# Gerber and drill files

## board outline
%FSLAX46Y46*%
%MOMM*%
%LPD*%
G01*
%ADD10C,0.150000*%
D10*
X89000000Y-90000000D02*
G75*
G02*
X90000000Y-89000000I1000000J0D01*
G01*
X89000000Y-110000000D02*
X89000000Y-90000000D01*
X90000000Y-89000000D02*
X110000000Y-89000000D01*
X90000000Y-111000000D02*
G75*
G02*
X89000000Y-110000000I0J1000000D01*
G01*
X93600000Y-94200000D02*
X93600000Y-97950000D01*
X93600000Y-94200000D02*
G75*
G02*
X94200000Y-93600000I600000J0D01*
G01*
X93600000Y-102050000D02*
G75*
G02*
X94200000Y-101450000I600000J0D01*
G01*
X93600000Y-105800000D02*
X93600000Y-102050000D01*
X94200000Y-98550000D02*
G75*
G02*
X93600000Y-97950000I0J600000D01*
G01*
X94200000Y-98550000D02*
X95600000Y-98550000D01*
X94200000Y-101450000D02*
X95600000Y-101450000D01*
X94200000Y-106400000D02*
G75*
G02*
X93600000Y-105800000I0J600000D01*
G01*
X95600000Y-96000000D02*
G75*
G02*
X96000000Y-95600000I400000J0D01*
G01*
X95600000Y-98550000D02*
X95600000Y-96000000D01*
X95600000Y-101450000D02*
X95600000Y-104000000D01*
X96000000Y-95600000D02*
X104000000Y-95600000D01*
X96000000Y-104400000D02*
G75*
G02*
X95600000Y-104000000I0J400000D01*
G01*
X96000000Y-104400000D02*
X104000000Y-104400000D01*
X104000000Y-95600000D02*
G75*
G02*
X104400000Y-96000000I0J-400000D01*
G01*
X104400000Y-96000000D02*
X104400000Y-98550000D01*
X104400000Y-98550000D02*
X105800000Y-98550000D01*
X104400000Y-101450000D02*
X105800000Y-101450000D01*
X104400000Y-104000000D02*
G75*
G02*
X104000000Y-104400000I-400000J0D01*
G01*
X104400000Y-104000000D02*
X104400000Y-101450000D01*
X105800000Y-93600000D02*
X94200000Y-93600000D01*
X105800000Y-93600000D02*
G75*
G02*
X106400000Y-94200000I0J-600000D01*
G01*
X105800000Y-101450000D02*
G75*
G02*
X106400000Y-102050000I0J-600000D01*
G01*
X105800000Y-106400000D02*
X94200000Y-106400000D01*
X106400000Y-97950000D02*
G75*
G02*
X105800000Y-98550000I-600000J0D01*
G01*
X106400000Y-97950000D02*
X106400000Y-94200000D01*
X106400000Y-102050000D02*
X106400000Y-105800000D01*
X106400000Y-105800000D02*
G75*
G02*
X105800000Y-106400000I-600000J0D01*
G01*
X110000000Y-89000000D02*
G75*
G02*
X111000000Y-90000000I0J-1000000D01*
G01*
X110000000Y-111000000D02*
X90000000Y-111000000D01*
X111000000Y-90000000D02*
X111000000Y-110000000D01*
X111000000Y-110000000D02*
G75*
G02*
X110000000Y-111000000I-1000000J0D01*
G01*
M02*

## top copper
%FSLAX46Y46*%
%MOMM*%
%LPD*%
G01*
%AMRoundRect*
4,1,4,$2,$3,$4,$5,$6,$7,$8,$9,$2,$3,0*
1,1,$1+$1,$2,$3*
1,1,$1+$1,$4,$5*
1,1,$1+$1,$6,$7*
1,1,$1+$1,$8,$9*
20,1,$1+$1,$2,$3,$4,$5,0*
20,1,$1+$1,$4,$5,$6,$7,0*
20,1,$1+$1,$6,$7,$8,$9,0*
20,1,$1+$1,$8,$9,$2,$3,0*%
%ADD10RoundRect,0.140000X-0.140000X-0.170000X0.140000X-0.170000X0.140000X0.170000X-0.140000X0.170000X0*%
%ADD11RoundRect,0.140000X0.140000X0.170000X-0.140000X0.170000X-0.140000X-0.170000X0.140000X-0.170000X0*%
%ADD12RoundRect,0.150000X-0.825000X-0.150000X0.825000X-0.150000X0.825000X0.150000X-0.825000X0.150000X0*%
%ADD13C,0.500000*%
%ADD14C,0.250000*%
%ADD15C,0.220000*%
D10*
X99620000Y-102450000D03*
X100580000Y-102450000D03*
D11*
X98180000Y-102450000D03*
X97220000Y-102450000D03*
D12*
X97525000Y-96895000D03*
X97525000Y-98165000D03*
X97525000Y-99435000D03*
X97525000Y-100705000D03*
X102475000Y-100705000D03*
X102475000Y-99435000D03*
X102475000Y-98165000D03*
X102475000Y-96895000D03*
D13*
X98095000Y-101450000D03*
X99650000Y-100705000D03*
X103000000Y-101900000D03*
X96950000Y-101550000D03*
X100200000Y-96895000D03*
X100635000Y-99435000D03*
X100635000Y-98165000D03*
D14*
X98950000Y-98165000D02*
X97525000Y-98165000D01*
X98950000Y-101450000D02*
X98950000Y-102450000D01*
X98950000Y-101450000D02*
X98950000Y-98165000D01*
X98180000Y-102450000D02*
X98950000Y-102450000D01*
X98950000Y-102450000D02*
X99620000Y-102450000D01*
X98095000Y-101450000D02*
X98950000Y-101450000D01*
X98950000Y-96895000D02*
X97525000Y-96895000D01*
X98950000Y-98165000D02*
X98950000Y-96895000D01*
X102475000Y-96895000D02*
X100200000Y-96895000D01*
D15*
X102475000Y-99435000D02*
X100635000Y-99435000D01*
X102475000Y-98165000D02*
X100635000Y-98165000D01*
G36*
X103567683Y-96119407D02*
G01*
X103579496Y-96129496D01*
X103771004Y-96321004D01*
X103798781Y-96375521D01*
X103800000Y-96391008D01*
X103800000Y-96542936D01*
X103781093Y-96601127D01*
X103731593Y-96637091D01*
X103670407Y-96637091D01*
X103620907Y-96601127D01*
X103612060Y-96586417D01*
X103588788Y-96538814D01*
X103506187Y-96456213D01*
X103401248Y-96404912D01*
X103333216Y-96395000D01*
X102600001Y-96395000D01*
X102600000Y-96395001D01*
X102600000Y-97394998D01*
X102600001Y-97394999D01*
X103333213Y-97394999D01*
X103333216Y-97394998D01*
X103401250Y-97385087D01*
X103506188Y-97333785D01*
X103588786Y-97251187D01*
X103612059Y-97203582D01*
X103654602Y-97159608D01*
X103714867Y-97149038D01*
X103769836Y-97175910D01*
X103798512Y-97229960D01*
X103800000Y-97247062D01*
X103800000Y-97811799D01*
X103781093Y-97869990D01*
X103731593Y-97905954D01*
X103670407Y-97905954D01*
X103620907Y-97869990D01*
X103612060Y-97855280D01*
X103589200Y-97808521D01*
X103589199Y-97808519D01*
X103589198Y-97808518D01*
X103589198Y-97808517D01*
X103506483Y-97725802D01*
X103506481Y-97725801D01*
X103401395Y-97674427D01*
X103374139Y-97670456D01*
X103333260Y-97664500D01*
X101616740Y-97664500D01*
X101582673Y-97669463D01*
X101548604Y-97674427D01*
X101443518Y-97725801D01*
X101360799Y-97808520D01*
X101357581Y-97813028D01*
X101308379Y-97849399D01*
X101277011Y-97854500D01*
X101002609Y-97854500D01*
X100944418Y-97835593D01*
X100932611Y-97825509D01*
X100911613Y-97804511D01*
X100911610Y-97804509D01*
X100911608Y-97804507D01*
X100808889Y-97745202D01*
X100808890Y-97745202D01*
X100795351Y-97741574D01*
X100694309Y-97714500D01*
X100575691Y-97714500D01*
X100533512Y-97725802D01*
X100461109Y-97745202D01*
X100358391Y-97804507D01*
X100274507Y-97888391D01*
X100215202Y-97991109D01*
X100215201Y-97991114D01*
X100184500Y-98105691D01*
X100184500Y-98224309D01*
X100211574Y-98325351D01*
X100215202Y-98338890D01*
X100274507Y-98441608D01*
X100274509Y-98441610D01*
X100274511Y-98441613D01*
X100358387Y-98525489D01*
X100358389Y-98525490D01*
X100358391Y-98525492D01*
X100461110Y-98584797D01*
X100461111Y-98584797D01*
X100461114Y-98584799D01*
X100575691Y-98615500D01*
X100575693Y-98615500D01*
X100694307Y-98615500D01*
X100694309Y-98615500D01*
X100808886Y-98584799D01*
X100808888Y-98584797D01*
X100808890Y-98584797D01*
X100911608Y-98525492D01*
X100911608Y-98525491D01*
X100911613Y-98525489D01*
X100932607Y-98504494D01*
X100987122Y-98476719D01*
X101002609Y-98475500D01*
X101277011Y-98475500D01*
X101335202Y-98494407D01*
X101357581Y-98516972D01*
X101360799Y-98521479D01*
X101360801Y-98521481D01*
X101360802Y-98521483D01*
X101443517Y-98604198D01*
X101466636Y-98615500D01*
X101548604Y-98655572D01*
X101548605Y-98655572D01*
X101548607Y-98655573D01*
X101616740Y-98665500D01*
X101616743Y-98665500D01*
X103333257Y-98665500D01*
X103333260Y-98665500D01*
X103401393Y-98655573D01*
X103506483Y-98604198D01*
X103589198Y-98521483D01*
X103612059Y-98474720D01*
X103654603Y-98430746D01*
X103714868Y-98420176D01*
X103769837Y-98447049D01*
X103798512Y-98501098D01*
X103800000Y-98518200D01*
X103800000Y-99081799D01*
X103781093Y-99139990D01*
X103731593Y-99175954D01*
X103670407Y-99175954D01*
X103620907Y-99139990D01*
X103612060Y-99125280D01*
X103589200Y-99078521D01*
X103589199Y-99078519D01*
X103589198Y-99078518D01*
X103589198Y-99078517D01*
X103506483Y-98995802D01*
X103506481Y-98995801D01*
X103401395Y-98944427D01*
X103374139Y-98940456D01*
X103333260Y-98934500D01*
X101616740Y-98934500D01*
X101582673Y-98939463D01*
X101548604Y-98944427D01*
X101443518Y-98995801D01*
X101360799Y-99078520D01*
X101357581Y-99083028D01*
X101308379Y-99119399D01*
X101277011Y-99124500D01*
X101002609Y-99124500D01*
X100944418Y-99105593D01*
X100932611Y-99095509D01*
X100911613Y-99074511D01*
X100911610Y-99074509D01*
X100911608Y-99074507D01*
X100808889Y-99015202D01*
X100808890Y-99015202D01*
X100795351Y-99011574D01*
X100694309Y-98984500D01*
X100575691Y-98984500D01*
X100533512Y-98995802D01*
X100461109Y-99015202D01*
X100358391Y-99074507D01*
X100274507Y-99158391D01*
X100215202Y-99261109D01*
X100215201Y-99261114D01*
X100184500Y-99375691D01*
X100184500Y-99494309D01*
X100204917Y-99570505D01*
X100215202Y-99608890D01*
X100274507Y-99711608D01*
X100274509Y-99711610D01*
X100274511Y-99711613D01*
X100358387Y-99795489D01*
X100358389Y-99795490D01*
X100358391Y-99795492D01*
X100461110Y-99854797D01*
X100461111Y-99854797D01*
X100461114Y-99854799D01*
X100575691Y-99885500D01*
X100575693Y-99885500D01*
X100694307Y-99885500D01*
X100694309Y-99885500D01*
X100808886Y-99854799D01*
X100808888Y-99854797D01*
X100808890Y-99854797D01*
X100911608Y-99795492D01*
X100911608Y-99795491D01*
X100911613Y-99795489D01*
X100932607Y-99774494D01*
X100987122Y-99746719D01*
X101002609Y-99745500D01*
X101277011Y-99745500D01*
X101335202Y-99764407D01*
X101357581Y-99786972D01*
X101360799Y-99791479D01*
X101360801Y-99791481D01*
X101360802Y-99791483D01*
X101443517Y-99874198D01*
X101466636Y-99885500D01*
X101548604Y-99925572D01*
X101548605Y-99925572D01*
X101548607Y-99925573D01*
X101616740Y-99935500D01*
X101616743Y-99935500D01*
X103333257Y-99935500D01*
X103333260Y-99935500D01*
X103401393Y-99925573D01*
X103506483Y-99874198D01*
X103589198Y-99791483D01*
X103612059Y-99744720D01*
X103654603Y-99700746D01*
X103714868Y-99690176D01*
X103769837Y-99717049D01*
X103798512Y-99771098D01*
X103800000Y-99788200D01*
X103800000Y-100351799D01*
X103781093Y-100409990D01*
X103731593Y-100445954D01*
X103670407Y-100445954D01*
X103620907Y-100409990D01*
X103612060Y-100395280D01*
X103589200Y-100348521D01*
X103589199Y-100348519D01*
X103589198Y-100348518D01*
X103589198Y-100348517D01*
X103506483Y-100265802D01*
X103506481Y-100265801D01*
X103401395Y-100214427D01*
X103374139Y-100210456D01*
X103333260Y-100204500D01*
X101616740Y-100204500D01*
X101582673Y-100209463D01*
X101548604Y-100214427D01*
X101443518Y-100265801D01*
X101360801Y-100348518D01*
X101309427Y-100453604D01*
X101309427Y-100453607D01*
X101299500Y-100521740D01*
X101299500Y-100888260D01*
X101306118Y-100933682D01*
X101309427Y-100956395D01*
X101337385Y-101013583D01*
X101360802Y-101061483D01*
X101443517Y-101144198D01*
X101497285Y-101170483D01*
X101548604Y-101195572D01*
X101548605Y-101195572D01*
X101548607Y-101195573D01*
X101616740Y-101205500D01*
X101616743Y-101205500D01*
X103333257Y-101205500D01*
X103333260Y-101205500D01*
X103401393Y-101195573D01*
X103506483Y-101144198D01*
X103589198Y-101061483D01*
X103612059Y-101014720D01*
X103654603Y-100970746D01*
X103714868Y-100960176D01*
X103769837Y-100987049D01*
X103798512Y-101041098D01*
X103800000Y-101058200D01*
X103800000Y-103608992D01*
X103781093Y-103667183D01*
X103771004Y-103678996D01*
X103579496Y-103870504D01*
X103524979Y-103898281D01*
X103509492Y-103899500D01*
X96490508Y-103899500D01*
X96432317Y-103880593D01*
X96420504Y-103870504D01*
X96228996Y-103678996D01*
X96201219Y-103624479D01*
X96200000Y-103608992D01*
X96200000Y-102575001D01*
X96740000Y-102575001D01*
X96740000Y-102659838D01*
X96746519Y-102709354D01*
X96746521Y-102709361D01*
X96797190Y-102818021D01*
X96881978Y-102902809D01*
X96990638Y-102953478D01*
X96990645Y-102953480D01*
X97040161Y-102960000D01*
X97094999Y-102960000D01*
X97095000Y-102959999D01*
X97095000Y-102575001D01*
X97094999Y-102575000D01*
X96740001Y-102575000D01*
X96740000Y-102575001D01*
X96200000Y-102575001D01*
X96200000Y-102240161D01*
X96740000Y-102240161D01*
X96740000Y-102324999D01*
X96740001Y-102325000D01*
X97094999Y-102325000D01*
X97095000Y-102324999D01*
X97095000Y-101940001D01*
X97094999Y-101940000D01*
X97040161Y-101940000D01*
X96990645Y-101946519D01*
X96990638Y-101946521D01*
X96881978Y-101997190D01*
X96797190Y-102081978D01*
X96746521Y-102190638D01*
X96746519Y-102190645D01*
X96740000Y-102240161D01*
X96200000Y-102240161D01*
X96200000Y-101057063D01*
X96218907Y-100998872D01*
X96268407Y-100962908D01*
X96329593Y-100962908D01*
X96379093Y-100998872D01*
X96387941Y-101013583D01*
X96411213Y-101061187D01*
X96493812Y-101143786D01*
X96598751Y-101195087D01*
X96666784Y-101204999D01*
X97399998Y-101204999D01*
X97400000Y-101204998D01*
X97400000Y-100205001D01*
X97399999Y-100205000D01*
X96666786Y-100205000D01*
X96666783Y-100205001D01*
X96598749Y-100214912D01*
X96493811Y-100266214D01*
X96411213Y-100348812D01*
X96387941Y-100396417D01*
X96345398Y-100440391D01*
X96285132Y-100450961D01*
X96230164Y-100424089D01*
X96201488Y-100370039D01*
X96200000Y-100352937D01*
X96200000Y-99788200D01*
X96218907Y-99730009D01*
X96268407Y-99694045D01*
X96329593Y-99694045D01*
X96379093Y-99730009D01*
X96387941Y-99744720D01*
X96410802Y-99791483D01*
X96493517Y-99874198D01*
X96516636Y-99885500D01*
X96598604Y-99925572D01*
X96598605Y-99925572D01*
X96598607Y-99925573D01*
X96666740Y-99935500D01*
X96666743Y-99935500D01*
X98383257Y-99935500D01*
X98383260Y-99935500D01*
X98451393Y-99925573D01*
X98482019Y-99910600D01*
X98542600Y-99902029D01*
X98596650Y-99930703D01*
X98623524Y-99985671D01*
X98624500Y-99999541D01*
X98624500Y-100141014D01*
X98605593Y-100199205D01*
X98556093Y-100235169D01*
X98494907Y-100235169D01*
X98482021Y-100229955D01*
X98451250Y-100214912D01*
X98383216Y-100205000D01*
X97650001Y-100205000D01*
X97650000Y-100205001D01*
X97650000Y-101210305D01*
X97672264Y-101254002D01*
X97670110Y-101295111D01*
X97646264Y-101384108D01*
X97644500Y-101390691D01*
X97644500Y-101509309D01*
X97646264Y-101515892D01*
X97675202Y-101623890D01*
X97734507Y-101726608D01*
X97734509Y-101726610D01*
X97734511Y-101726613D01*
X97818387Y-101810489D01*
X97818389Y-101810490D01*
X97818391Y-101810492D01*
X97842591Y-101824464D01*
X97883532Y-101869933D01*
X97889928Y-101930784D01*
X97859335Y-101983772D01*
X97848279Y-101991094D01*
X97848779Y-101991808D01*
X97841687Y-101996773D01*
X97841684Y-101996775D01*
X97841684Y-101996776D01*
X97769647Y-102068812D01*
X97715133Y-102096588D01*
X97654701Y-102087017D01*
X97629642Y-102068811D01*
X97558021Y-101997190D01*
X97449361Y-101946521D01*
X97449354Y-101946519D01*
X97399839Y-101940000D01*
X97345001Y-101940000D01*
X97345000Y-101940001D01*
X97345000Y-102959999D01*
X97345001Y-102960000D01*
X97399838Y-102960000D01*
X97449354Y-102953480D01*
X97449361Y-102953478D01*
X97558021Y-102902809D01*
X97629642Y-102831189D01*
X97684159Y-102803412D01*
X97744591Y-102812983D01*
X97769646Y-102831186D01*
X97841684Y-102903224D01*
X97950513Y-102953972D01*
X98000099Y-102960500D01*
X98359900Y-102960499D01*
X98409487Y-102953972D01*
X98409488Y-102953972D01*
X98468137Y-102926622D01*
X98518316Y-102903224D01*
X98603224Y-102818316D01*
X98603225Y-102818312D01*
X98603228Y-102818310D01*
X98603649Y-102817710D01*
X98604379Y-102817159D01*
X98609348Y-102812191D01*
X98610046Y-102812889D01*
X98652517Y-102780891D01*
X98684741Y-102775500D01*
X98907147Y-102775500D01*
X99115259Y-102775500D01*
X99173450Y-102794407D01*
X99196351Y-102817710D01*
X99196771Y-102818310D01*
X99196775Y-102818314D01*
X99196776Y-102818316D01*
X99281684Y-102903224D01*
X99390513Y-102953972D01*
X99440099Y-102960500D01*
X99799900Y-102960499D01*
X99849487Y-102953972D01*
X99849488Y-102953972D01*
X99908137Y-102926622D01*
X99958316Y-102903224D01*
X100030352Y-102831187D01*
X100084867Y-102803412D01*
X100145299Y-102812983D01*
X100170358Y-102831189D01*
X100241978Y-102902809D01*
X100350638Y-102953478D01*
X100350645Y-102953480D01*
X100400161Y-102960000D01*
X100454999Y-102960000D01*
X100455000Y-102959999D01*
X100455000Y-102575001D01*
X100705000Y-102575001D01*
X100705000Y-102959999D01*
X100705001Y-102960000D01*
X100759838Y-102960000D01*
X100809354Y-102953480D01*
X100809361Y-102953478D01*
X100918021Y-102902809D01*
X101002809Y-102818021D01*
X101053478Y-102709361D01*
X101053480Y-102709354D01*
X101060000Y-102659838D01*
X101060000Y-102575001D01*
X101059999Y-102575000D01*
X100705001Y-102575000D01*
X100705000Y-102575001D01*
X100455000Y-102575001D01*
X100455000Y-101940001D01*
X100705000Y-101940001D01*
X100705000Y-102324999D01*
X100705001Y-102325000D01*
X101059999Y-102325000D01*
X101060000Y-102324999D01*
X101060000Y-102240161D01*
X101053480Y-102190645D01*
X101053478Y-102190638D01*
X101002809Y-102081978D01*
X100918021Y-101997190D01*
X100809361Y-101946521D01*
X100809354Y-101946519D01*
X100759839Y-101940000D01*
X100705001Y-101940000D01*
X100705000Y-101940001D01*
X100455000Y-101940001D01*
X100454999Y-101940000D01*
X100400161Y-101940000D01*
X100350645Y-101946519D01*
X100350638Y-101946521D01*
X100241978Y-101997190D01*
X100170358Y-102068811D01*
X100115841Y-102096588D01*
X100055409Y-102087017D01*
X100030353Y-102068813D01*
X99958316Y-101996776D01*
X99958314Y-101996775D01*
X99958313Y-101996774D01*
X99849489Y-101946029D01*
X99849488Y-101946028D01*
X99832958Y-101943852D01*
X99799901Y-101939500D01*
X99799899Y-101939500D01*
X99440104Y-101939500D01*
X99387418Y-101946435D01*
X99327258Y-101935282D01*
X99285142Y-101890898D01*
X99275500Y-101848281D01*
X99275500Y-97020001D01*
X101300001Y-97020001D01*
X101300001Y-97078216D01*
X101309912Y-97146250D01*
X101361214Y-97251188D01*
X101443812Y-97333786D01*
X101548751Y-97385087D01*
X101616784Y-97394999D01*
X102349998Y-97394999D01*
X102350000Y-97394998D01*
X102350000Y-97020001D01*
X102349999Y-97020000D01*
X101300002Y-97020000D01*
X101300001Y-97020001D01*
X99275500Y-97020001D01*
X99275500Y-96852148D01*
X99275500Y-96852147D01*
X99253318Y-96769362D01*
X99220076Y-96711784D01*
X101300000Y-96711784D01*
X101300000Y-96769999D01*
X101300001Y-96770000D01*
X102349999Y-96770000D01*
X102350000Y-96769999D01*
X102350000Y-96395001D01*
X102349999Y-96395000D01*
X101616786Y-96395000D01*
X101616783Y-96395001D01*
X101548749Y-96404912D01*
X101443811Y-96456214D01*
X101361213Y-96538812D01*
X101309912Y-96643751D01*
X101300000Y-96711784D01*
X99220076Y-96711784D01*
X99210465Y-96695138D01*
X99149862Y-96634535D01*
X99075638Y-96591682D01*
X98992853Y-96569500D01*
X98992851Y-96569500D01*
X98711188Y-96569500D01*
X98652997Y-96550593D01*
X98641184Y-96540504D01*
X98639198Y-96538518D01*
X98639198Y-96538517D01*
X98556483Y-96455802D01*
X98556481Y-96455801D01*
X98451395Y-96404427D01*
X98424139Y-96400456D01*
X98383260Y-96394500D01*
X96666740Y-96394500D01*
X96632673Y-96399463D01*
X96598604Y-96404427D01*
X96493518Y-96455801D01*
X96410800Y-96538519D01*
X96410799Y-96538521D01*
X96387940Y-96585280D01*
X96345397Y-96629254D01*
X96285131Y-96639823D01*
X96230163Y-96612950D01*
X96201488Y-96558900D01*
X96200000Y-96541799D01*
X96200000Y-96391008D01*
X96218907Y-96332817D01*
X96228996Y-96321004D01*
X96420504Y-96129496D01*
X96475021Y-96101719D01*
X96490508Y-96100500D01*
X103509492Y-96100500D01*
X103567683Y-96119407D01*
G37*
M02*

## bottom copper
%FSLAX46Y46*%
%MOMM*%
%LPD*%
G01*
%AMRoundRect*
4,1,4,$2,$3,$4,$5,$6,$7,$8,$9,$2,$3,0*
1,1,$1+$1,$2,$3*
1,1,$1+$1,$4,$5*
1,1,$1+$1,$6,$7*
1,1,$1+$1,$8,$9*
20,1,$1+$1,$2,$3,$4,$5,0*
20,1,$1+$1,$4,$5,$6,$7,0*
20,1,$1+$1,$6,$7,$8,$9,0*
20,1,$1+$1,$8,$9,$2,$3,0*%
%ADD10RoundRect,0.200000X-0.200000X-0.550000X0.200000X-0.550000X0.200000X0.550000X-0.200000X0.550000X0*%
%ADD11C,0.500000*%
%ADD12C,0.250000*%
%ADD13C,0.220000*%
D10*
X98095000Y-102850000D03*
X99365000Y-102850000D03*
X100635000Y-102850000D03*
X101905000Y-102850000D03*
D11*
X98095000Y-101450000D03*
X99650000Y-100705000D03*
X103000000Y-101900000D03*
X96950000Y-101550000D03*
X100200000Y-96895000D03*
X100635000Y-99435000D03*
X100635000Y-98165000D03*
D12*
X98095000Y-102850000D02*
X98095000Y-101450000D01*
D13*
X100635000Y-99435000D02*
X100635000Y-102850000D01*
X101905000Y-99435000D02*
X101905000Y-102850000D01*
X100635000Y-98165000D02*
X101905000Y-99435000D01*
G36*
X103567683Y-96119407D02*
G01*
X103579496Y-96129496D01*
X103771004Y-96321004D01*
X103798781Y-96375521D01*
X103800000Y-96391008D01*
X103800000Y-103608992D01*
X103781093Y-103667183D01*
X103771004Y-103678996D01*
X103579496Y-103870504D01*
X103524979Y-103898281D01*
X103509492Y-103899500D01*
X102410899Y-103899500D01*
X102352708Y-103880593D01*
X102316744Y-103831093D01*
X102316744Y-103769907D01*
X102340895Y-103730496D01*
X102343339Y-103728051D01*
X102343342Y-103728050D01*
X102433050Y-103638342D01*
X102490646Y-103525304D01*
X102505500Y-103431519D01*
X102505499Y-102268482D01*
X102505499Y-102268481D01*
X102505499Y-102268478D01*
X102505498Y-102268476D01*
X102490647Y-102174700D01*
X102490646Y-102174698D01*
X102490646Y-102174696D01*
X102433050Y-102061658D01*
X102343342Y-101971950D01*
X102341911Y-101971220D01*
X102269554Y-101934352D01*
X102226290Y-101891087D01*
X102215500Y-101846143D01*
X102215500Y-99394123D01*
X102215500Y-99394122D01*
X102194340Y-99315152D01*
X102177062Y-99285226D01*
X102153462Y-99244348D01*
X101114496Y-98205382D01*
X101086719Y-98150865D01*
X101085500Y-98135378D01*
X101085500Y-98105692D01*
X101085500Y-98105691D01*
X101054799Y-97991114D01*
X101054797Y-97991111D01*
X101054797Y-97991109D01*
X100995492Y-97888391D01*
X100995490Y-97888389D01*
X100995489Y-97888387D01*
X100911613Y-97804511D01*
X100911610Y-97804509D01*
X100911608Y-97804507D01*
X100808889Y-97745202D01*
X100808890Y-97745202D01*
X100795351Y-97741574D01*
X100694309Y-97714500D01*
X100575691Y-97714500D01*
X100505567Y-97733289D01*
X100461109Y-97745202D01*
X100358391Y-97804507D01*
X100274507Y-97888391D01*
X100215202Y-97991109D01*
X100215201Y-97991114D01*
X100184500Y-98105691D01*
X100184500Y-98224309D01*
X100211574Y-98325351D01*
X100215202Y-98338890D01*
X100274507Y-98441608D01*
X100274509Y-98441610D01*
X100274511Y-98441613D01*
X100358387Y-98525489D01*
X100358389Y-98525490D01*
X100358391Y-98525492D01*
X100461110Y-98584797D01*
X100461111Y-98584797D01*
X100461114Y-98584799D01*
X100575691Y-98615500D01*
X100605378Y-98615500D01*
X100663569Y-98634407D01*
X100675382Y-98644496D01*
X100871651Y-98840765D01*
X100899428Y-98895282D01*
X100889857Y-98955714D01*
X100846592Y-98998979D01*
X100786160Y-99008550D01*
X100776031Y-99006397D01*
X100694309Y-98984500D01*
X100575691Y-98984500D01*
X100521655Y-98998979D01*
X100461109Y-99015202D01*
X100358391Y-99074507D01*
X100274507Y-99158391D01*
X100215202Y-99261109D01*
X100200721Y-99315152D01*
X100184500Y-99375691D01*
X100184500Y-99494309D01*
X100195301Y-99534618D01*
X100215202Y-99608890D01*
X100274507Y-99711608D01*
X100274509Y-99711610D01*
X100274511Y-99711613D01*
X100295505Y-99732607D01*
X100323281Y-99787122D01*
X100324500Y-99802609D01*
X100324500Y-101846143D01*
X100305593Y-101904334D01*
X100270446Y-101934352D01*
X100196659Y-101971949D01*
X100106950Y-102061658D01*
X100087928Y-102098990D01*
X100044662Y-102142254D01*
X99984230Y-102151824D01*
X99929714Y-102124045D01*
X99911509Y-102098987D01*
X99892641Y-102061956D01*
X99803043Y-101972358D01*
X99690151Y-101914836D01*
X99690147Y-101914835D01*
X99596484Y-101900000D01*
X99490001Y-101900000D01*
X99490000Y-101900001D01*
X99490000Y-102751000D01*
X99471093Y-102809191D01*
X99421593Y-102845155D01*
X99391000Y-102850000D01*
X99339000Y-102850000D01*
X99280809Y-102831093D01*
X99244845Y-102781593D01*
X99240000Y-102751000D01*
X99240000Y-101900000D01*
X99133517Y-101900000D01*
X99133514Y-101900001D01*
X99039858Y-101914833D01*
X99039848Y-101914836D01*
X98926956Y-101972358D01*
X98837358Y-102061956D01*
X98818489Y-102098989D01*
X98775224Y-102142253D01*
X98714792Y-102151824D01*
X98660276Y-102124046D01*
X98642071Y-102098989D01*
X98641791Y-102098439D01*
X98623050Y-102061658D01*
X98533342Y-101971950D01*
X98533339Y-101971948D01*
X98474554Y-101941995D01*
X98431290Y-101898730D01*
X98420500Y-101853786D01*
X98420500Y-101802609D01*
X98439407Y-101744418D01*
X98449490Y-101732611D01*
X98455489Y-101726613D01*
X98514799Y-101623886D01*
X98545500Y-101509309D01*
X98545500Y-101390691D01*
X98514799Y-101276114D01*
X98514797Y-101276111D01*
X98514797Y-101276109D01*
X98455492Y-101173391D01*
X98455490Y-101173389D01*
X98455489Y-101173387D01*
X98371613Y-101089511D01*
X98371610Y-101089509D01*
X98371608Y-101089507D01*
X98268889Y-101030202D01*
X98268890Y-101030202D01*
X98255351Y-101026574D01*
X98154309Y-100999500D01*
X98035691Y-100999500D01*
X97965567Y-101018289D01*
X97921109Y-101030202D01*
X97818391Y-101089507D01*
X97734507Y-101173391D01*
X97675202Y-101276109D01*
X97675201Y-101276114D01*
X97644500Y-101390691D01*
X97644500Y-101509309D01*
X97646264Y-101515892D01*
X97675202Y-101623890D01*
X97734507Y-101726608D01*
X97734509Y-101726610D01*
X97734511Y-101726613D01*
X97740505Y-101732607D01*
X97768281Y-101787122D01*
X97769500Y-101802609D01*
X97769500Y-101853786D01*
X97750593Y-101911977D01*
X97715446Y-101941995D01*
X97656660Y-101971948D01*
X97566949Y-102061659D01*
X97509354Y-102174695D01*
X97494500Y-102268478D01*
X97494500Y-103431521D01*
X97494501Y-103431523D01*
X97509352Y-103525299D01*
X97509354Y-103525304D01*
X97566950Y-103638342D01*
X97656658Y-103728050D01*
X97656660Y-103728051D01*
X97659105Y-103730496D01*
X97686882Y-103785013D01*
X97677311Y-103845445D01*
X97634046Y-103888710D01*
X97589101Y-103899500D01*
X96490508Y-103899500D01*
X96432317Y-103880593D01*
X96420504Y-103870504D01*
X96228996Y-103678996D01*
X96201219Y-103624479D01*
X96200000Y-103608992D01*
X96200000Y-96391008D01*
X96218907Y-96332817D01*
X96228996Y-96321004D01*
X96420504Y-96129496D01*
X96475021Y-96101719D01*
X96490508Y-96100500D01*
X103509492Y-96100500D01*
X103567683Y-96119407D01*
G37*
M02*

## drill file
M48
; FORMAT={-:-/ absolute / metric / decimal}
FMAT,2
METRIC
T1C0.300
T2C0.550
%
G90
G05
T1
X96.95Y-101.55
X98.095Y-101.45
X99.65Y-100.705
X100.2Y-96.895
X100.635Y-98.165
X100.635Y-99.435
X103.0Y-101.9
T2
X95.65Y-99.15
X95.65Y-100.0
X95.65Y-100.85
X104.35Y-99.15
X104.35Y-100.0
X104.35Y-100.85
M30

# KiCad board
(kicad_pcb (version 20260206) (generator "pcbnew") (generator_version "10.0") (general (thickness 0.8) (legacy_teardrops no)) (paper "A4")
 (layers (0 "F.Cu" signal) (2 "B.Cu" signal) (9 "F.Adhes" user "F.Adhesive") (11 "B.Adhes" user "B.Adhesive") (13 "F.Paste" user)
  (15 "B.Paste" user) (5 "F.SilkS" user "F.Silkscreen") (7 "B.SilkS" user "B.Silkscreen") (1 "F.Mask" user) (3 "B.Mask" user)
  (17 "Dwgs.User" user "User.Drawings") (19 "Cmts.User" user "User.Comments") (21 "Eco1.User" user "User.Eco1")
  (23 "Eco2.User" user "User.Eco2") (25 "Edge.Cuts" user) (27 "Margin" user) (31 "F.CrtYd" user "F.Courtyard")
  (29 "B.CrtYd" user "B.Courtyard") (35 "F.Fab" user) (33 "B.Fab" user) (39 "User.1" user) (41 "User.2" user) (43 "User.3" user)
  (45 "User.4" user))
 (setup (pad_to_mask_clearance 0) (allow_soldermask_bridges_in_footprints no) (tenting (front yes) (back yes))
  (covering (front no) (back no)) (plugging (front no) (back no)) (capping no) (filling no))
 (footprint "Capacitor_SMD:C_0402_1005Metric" (layer "F.Cu") (at 100.1 102.45)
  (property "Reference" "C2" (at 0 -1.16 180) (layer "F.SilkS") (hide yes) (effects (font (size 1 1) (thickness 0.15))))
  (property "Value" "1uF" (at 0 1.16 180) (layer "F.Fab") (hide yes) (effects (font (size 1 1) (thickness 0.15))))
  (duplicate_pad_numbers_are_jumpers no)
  (pad "1" smd roundrect (at -0.48 0) (size 0.56 0.62) (layers "F.Cu" "F.Mask" "F.Paste") (roundrect_rratio 0.25) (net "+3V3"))
  (pad "2" smd roundrect (at 0.48 0) (size 0.56 0.62) (layers "F.Cu" "F.Mask" "F.Paste") (roundrect_rratio 0.25) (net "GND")))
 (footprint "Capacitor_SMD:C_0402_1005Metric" (layer "F.Cu") (at 97.7 102.45 180)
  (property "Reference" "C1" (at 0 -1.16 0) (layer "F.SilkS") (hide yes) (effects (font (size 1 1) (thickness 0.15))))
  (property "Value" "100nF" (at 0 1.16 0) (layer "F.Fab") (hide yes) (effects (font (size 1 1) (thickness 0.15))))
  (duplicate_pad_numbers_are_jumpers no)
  (pad "1" smd roundrect (at -0.48 0 180) (size 0.56 0.62) (layers "F.Cu" "F.Mask" "F.Paste") (roundrect_rratio 0.25) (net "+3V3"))
  (pad "2" smd roundrect (at 0.48 0 180) (size 0.56 0.62) (layers "F.Cu" "F.Mask" "F.Paste") (roundrect_rratio 0.25) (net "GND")))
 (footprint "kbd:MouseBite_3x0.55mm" (layer "F.Cu") (at 104.35 100)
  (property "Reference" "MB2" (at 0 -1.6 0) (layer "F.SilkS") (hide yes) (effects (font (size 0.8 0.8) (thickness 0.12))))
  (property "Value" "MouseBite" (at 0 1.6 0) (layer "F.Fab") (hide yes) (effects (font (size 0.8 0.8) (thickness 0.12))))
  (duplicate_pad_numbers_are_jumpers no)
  (pad "" np_thru_hole circle (at 0 -0.85) (size 0.55 0.55) (drill 0.55) (layers "*.Cu" "*.Mask"))
  (pad "" np_thru_hole circle (at 0 0) (size 0.55 0.55) (drill 0.55) (layers "*.Cu" "*.Mask"))
  (pad "" np_thru_hole circle (at 0 0.85) (size 0.55 0.55) (drill 0.55) (layers "*.Cu" "*.Mask")))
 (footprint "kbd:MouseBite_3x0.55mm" (layer "F.Cu") (at 95.65 100)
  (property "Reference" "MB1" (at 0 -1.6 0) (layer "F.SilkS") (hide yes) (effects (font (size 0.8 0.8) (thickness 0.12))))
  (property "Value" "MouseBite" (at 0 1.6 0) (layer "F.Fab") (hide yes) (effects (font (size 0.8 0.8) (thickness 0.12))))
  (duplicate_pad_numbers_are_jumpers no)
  (pad "" np_thru_hole circle (at 0 -0.85) (size 0.55 0.55) (drill 0.55) (layers "*.Cu" "*.Mask"))
  (pad "" np_thru_hole circle (at 0 0) (size 0.55 0.55) (drill 0.55) (layers "*.Cu" "*.Mask"))
  (pad "" np_thru_hole circle (at 0 0.85) (size 0.55 0.55) (drill 0.55) (layers "*.Cu" "*.Mask")))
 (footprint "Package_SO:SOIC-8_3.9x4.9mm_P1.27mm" (layer "F.Cu") (at 100 98.8)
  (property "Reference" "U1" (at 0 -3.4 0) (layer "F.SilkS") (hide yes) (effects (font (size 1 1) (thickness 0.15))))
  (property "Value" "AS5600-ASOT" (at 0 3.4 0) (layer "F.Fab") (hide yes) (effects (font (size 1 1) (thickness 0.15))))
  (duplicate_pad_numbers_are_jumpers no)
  (pad "1" smd roundrect (at -2.475 -1.905) (size 1.95 0.6) (layers "F.Cu" "F.Mask" "F.Paste") (roundrect_rratio 0.25) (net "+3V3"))
  (pad "2" smd roundrect (at -2.475 -0.635) (size 1.95 0.6) (layers "F.Cu" "F.Mask" "F.Paste") (roundrect_rratio 0.25) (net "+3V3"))
  (pad "3" smd roundrect (at -2.475 0.635) (size 1.95 0.6) (layers "F.Cu" "F.Mask" "F.Paste") (roundrect_rratio 0.25)
   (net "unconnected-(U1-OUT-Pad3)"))
  (pad "4" smd roundrect (at -2.475 1.905) (size 1.95 0.6) (layers "F.Cu" "F.Mask" "F.Paste") (roundrect_rratio 0.25) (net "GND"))
  (pad "5" smd roundrect (at 2.475 1.905) (size 1.95 0.6) (layers "F.Cu" "F.Mask" "F.Paste") (roundrect_rratio 0.25)
   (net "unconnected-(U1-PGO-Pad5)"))
  (pad "6" smd roundrect (at 2.475 0.635) (size 1.95 0.6) (layers "F.Cu" "F.Mask" "F.Paste") (roundrect_rratio 0.25) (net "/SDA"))
  (pad "7" smd roundrect (at 2.475 -0.635) (size 1.95 0.6) (layers "F.Cu" "F.Mask" "F.Paste") (roundrect_rratio 0.25) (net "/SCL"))
  (pad "8" smd roundrect (at 2.475 -1.905) (size 1.95 0.6) (layers "F.Cu" "F.Mask" "F.Paste") (roundrect_rratio 0.25) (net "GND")))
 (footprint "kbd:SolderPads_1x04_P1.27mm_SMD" (layer "B.Cu") (at 100 102.85)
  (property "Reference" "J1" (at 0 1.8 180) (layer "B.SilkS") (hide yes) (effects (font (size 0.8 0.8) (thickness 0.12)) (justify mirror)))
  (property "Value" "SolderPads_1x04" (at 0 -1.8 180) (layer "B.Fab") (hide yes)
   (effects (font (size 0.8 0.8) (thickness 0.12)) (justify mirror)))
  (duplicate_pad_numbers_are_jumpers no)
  (pad "1" smd roundrect (at -1.905 0) (size 0.8 1.5) (layers "B.Cu" "B.Mask" "B.Paste") (roundrect_rratio 0.25) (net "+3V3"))
  (pad "2" smd roundrect (at -0.635 0) (size 0.8 1.5) (layers "B.Cu" "B.Mask" "B.Paste") (roundrect_rratio 0.25) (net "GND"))
  (pad "3" smd roundrect (at 0.635 0) (size 0.8 1.5) (layers "B.Cu" "B.Mask" "B.Paste") (roundrect_rratio 0.25) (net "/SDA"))
  (pad "4" smd roundrect (at 1.905 0) (size 0.8 1.5) (layers "B.Cu" "B.Mask" "B.Paste") (roundrect_rratio 0.25) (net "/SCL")))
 (gr_arc (start 89 90) (mid 89.292893 89.292893) (end 90 89) (stroke (width 0.15) (type default)) (layer "Edge.Cuts"))
 (gr_line (start 89 110) (end 89 90) (stroke (width 0.15) (type default)) (layer "Edge.Cuts"))
 (gr_line (start 90 89) (end 110 89) (stroke (width 0.15) (type default)) (layer "Edge.Cuts"))
 (gr_arc (start 90 111) (mid 89.292893 110.707107) (end 89 110) (stroke (width 0.15) (type default)) (layer "Edge.Cuts"))
 (gr_line (start 93.6 94.2) (end 93.6 97.95) (stroke (width 0.15) (type default)) (layer "Edge.Cuts"))
 (gr_arc (start 93.6 94.2) (mid 93.775736 93.775736) (end 94.2 93.6) (stroke (width 0.15) (type default)) (layer "Edge.Cuts"))
 (gr_arc (start 93.6 102.05) (mid 93.775736 101.625736) (end 94.2 101.45) (stroke (width 0.15) (type default)) (layer "Edge.Cuts"))
 (gr_line (start 93.6 105.8) (end 93.6 102.05) (stroke (width 0.15) (type default)) (layer "Edge.Cuts"))
 (gr_arc (start 94.2 98.55) (mid 93.775736 98.374264) (end 93.6 97.95) (stroke (width 0.15) (type default)) (layer "Edge.Cuts"))
 (gr_line (start 94.2 98.55) (end 95.6 98.55) (stroke (width 0.15) (type default)) (layer "Edge.Cuts"))
 (gr_line (start 94.2 101.45) (end 95.6 101.45) (stroke (width 0.15) (type default)) (layer "Edge.Cuts"))
 (gr_arc (start 94.2 106.4) (mid 93.775736 106.224264) (end 93.6 105.8) (stroke (width 0.15) (type default)) (layer "Edge.Cuts"))
 (gr_arc (start 95.6 96) (mid 95.717157 95.717157) (end 96 95.6) (stroke (width 0.15) (type default)) (layer "Edge.Cuts"))
 (gr_line (start 95.6 98.55) (end 95.6 96) (stroke (width 0.15) (type default)) (layer "Edge.Cuts"))
 (gr_line (start 95.6 101.45) (end 95.6 104) (stroke (width 0.15) (type default)) (layer "Edge.Cuts"))
 (gr_line (start 96 95.6) (end 104 95.6) (stroke (width 0.15) (type default)) (layer "Edge.Cuts"))
 (gr_arc (start 96 104.4) (mid 95.717157 104.282843) (end 95.6 104) (stroke (width 0.15) (type default)) (layer "Edge.Cuts"))
 (gr_line (start 96 104.4) (end 104 104.4) (stroke (width 0.15) (type default)) (layer "Edge.Cuts"))
 (gr_arc (start 104 95.6) (mid 104.282843 95.717157) (end 104.4 96) (stroke (width 0.15) (type default)) (layer "Edge.Cuts"))
 (gr_line (start 104.4 96) (end 104.4 98.55) (stroke (width 0.15) (type default)) (layer "Edge.Cuts"))
 (gr_line (start 104.4 98.55) (end 105.8 98.55) (stroke (width 0.15) (type default)) (layer "Edge.Cuts"))
 (gr_line (start 104.4 101.45) (end 105.8 101.45) (stroke (width 0.15) (type default)) (layer "Edge.Cuts"))
 (gr_arc (start 104.4 104) (mid 104.282843 104.282843) (end 104 104.4) (stroke (width 0.15) (type default)) (layer "Edge.Cuts"))
 (gr_line (start 104.4 104) (end 104.4 101.45) (stroke (width 0.15) (type default)) (layer "Edge.Cuts"))
 (gr_line (start 105.8 93.6) (end 94.2 93.6) (stroke (width 0.15) (type default)) (layer "Edge.Cuts"))
 (gr_arc (start 105.8 93.6) (mid 106.224264 93.775736) (end 106.4 94.2) (stroke (width 0.15) (type default)) (layer "Edge.Cuts"))
 (gr_arc (start 105.8 101.45) (mid 106.224264 101.625736) (end 106.4 102.05) (stroke (width 0.15) (type default)) (layer "Edge.Cuts"))
 (gr_line (start 105.8 106.4) (end 94.2 106.4) (stroke (width 0.15) (type default)) (layer "Edge.Cuts"))
 (gr_arc (start 106.4 97.95) (mid 106.224264 98.374264) (end 105.8 98.55) (stroke (width 0.15) (type default)) (layer "Edge.Cuts"))
 (gr_line (start 106.4 97.95) (end 106.4 94.2) (stroke (width 0.15) (type default)) (layer "Edge.Cuts"))
 (gr_line (start 106.4 102.05) (end 106.4 105.8) (stroke (width 0.15) (type default)) (layer "Edge.Cuts"))
 (gr_arc (start 106.4 105.8) (mid 106.224264 106.224264) (end 105.8 106.4) (stroke (width 0.15) (type default)) (layer "Edge.Cuts"))
 (gr_arc (start 110 89) (mid 110.707107 89.292893) (end 111 90) (stroke (width 0.15) (type default)) (layer "Edge.Cuts"))
 (gr_line (start 110 111) (end 90 111) (stroke (width 0.15) (type default)) (layer "Edge.Cuts"))
 (gr_line (start 111 90) (end 111 110) (stroke (width 0.15) (type default)) (layer "Edge.Cuts"))
 (gr_arc (start 111 110) (mid 110.707107 110.707107) (end 110 111) (stroke (width 0.15) (type default)) (layer "Edge.Cuts"))
 (segment (start 98.95 98.165) (end 97.525 98.165) (width 0.25) (layer "F.Cu") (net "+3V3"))
 (segment (start 98.95 101.45) (end 98.95 102.45) (width 0.25) (layer "F.Cu") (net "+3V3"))
 (segment (start 98.95 101.45) (end 98.95 98.165) (width 0.25) (layer "F.Cu") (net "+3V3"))
 (segment (start 98.18 102.45) (end 98.95 102.45) (width 0.25) (layer "F.Cu") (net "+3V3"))
 (segment (start 98.95 102.45) (end 99.62 102.45) (width 0.25) (layer "F.Cu") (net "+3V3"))
 (segment (start 98.095 101.45) (end 98.95 101.45) (width 0.25) (layer "F.Cu") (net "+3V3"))
 (segment (start 98.95 96.895) (end 97.525 96.895) (width 0.25) (layer "F.Cu") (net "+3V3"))
 (segment (start 98.95 98.165) (end 98.95 96.895) (width 0.25) (layer "F.Cu") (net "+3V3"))
 (via (at 98.095 101.45) (size 0.5) (drill 0.3) (layers "F.Cu" "B.Cu") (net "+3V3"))
 (segment (start 98.095 102.85) (end 98.095 101.45) (width 0.25) (layer "B.Cu") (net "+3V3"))
 (segment (start 102.475 96.895) (end 100.2 96.895) (width 0.25) (layer "F.Cu") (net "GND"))
 (via (at 99.65 100.705) (size 0.5) (drill 0.3) (layers "F.Cu" "B.Cu") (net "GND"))
 (via (at 103 101.9) (size 0.5) (drill 0.3) (layers "F.Cu" "B.Cu") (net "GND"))
 (via (at 96.95 101.55) (size 0.5) (drill 0.3) (layers "F.Cu" "B.Cu") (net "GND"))
 (via (at 100.2 96.895) (size 0.5) (drill 0.3) (layers "F.Cu" "B.Cu") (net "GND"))
 (segment (start 102.475 99.435) (end 100.635 99.435) (width 0.22) (layer "F.Cu") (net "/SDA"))
 (via (at 100.635 99.435) (size 0.5) (drill 0.3) (layers "F.Cu" "B.Cu") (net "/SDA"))
 (segment (start 100.635 99.435) (end 100.635 102.85) (width 0.22) (layer "B.Cu") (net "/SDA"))
 (segment (start 102.475 98.165) (end 100.635 98.165) (width 0.22) (layer "F.Cu") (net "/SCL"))
 (via (at 100.635 98.165) (size 0.5) (drill 0.3) (layers "F.Cu" "B.Cu") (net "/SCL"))
 (segment (start 101.905 99.435) (end 101.905 102.85) (width 0.22) (layer "B.Cu") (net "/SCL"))
 (segment (start 100.635 98.165) (end 101.905 99.435) (width 0.22) (layer "B.Cu") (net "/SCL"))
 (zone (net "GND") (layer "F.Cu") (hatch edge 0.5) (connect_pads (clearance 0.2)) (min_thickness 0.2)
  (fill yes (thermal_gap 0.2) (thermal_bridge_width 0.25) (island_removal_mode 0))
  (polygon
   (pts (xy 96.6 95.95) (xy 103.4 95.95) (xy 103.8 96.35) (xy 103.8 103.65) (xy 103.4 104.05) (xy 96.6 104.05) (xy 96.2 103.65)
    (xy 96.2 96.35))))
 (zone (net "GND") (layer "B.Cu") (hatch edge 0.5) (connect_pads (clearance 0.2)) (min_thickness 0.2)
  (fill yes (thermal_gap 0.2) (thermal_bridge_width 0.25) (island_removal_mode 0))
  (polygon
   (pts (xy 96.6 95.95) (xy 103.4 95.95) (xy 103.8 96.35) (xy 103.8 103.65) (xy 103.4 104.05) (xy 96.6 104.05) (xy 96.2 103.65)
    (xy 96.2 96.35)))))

